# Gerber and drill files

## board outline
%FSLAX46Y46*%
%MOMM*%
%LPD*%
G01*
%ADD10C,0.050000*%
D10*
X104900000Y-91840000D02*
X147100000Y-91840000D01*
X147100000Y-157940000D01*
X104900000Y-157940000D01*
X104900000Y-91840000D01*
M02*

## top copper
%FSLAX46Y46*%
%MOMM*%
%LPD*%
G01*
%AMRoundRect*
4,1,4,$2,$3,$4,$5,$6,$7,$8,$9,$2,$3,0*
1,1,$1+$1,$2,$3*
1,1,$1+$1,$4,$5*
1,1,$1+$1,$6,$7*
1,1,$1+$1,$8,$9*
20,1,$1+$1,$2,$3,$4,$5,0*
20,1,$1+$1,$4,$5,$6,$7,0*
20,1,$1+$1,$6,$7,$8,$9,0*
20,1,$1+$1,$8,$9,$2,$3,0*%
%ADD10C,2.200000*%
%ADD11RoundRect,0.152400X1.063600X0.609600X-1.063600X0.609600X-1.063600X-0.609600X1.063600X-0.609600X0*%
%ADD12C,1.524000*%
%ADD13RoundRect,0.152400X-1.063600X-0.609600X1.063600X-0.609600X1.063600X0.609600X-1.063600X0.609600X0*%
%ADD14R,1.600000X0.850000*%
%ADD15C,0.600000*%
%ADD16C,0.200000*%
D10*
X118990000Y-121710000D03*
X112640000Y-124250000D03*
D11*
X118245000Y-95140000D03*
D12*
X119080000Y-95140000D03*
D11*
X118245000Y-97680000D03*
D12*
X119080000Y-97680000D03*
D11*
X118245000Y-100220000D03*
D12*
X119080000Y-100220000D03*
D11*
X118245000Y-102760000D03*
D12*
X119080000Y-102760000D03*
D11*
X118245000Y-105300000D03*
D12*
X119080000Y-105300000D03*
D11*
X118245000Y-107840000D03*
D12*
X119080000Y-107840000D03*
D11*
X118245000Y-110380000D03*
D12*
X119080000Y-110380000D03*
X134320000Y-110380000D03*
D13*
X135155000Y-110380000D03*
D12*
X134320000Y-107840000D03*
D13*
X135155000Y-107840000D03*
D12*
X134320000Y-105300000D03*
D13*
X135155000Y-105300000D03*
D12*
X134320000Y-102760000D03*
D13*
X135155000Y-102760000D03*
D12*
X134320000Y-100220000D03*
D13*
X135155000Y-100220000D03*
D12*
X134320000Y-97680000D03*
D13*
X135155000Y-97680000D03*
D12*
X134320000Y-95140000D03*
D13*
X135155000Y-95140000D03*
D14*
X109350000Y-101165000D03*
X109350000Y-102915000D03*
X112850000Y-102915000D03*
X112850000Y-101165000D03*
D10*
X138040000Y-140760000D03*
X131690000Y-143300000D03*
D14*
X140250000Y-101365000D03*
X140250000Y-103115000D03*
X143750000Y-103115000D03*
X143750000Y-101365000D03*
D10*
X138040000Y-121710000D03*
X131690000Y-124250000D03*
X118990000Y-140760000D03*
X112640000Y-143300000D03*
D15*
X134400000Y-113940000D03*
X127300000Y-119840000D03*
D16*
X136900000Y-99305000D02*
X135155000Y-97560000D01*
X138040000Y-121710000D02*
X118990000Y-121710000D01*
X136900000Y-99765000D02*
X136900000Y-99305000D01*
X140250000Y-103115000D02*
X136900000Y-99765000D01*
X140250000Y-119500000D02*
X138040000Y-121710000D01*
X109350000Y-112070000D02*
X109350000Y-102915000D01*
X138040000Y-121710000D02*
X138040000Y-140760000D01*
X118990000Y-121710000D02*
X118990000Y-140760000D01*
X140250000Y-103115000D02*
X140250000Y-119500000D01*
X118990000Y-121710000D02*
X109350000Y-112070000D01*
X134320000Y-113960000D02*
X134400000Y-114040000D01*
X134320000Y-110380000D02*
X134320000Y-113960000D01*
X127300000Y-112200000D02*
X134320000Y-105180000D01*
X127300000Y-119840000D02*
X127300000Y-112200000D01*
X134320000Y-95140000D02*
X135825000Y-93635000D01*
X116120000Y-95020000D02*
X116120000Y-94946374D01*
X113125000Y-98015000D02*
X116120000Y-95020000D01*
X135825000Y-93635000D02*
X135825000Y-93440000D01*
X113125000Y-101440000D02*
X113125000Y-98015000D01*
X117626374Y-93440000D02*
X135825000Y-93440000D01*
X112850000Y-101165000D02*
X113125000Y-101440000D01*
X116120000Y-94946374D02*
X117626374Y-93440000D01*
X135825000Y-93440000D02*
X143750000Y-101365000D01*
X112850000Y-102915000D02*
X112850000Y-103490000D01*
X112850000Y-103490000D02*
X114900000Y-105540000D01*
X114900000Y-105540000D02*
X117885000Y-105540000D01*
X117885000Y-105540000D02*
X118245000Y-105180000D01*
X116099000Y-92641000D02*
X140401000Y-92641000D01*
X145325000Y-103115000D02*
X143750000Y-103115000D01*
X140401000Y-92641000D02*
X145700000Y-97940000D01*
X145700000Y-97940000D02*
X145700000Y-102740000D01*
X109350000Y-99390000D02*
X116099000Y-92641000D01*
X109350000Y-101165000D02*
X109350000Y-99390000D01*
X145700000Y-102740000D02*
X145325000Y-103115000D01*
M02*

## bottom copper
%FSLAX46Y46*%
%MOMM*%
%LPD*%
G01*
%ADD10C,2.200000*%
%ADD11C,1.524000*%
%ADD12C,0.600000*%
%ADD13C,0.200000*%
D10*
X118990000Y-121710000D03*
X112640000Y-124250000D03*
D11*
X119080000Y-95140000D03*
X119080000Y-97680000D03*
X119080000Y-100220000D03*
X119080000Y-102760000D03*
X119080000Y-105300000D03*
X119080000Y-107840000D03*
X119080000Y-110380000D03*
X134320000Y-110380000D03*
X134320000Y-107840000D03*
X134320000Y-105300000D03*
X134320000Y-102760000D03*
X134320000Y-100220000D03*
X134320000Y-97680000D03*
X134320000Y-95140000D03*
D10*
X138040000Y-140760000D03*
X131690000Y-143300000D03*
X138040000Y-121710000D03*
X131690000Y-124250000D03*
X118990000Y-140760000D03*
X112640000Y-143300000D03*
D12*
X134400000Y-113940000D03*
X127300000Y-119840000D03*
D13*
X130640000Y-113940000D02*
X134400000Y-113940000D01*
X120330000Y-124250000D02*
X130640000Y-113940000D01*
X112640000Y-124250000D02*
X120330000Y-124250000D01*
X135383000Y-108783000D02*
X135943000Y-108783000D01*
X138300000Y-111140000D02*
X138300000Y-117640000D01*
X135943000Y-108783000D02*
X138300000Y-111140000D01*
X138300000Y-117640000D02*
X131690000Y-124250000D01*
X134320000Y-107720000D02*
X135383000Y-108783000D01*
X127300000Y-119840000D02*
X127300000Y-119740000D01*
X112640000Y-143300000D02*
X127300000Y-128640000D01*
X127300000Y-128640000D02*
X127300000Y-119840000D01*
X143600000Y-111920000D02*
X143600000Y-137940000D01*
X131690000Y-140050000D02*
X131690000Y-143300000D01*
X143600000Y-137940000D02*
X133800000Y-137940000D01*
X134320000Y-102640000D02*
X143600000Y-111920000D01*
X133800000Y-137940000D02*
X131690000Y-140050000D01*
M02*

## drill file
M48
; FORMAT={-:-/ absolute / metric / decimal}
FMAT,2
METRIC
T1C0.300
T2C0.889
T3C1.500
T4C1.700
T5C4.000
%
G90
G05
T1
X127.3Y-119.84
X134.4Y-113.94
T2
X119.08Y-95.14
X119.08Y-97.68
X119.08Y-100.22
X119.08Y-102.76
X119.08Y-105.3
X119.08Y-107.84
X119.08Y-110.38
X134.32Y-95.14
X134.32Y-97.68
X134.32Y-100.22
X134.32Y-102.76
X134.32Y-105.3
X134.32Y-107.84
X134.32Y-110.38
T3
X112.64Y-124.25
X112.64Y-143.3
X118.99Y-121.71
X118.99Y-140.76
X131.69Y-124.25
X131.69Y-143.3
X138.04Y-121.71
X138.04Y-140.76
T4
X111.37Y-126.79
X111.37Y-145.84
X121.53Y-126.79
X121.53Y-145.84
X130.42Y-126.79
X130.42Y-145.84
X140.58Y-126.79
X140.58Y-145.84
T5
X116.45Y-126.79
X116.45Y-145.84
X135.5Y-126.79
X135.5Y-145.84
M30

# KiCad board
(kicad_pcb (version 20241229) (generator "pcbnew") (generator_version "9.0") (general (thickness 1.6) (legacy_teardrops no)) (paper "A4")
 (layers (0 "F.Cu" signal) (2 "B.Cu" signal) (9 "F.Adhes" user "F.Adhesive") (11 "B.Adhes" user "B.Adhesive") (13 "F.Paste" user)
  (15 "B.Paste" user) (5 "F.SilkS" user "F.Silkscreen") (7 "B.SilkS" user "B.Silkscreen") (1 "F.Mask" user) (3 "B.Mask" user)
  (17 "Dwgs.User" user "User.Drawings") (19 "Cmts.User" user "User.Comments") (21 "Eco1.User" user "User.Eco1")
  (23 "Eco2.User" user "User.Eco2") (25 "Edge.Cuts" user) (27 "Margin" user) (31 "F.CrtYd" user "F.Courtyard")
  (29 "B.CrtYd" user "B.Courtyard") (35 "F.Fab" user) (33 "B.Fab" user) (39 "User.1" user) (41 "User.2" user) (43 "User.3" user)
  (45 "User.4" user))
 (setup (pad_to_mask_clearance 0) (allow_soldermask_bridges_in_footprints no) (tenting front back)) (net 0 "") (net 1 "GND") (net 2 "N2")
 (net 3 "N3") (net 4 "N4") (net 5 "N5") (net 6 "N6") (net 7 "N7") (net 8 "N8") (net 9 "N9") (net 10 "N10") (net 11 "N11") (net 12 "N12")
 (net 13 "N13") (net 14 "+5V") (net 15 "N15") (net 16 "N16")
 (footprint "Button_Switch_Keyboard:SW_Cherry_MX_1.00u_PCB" (layer "F.Cu") (at 118.99 121.71)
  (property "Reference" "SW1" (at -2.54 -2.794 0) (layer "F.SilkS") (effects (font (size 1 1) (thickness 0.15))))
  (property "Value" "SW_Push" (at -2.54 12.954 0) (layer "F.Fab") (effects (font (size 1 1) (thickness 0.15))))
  (pad "" np_thru_hole circle (at -7.62 5.08) (size 1.7 1.7) (drill 1.7) (layers "*.Cu" "*.Mask"))
  (pad "" np_thru_hole circle (at -2.54 5.08) (size 4 4) (drill 4) (layers "*.Cu" "*.Mask"))
  (pad "" np_thru_hole circle (at 2.54 5.08) (size 1.7 1.7) (drill 1.7) (layers "*.Cu" "*.Mask"))
  (pad "1" thru_hole circle (at 0 0) (size 2.2 2.2) (drill 1.5) (layers "*.Cu" "*.Mask") (remove_unused_layers no) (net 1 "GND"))
  (pad "2" thru_hole circle (at -6.35 2.54) (size 2.2 2.2) (drill 1.5) (layers "*.Cu" "*.Mask") (remove_unused_layers no) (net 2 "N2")))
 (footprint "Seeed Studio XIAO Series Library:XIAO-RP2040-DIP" (layer "F.Cu") (at 126.7 102.76)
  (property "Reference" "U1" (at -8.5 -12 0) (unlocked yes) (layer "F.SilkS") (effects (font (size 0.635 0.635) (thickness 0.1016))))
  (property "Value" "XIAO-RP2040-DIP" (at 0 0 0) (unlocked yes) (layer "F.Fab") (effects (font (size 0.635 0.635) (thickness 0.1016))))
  (pad "1" smd roundrect (at -8.455 -7.62 180) (size 2.432 1.524) (layers "F.Cu" "F.Mask") (roundrect_rratio 0.1) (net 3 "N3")
   (thermal_bridge_angle 45))
  (pad "1" thru_hole circle (at -7.62 -7.62 180) (size 1.524 1.524) (drill 0.889) (layers "*.Cu" "*.Mask") (remove_unused_layers no)
   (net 3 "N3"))
  (pad "2" smd roundrect (at -8.455 -5.08 180) (size 2.432 1.524) (layers "F.Cu" "F.Mask") (roundrect_rratio 0.1) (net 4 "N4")
   (thermal_bridge_angle 45))
  (pad "2" thru_hole circle (at -7.62 -5.08 180) (size 1.524 1.524) (drill 0.889) (layers "*.Cu" "*.Mask") (remove_unused_layers no)
   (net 4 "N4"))
  (pad "3" smd roundrect (at -8.455 -2.54 180) (size 2.432 1.524) (layers "F.Cu" "F.Mask") (roundrect_rratio 0.1) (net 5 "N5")
   (thermal_bridge_angle 45))
  (pad "3" thru_hole circle (at -7.62 -2.54 180) (size 1.524 1.524) (drill 0.889) (layers "*.Cu" "*.Mask") (remove_unused_layers no)
   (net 5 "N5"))
  (pad "4" smd roundrect (at -8.455 0 180) (size 2.432 1.524) (layers "F.Cu" "F.Mask") (roundrect_rratio 0.1) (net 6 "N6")
   (thermal_bridge_angle 45))
  (pad "4" thru_hole circle (at -7.62 0 180) (size 1.524 1.524) (drill 0.889) (layers "*.Cu" "*.Mask") (remove_unused_layers no)
   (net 6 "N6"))
  (pad "5" smd roundrect (at -8.455 2.54 180) (size 2.432 1.524) (layers "F.Cu" "F.Mask") (roundrect_rratio 0.1) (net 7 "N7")
   (thermal_bridge_angle 45))
  (pad "5" thru_hole circle (at -7.62 2.54 180) (size 1.524 1.524) (drill 0.889) (layers "*.Cu" "*.Mask") (remove_unused_layers no)
   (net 7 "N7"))
  (pad "6" smd roundrect (at -8.455 5.08 180) (size 2.432 1.524) (layers "F.Cu" "F.Mask") (roundrect_rratio 0.1) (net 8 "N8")
   (thermal_bridge_angle 45))
  (pad "6" thru_hole circle (at -7.62 5.08 180) (size 1.524 1.524) (drill 0.889) (layers "*.Cu" "*.Mask") (remove_unused_layers no)
   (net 8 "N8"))
  (pad "7" smd roundrect (at -8.455 7.62 180) (size 2.432 1.524) (layers "F.Cu" "F.Mask") (roundrect_rratio 0.1) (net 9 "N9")
   (thermal_bridge_angle 45))
  (pad "7" thru_hole circle (at -7.62 7.62 180) (size 1.524 1.524) (drill 0.889) (layers "*.Cu" "*.Mask") (remove_unused_layers no)
   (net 9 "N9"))
  (pad "8" thru_hole circle (at 7.62 7.62) (size 1.524 1.524) (drill 0.889) (layers "*.Cu" "*.Mask") (remove_unused_layers no) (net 2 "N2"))
  (pad "8" smd roundrect (at 8.455 7.62) (size 2.432 1.524) (layers "F.Cu" "F.Mask") (roundrect_rratio 0.1) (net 2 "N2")
   (thermal_bridge_angle 45))
  (pad "9" thru_hole circle (at 7.62 5.08) (size 1.524 1.524) (drill 0.889) (layers "*.Cu" "*.Mask") (remove_unused_layers no)
   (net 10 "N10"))
  (pad "9" smd roundrect (at 8.455 5.08) (size 2.432 1.524) (layers "F.Cu" "F.Mask") (roundrect_rratio 0.1) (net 10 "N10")
   (thermal_bridge_angle 45))
  (pad "10" thru_hole circle (at 7.62 2.54) (size 1.524 1.524) (drill 0.889) (layers "*.Cu" "*.Mask") (remove_unused_layers no)
   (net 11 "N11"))
  (pad "10" smd roundrect (at 8.455 2.54) (size 2.432 1.524) (layers "F.Cu" "F.Mask") (roundrect_rratio 0.1) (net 11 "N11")
   (thermal_bridge_angle 45))
  (pad "11" thru_hole circle (at 7.62 0) (size 1.524 1.524) (drill 0.889) (layers "*.Cu" "*.Mask") (remove_unused_layers no) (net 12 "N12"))
  (pad "11" smd roundrect (at 8.455 0) (size 2.432 1.524) (layers "F.Cu" "F.Mask") (roundrect_rratio 0.1) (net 12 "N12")
   (thermal_bridge_angle 45))
  (pad "12" thru_hole circle (at 7.62 -2.54) (size 1.524 1.524) (drill 0.889) (layers "*.Cu" "*.Mask") (remove_unused_layers no)
   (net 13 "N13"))
  (pad "12" smd roundrect (at 8.455 -2.54) (size 2.432 1.524) (layers "F.Cu" "F.Mask") (roundrect_rratio 0.1) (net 13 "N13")
   (thermal_bridge_angle 45))
  (pad "13" thru_hole circle (at 7.62 -5.08) (size 1.524 1.524) (drill 0.889) (layers "*.Cu" "*.Mask") (remove_unused_layers no)
   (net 1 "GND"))
  (pad "13" smd roundrect (at 8.455 -5.08) (size 2.432 1.524) (layers "F.Cu" "F.Mask") (roundrect_rratio 0.1) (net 1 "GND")
   (thermal_bridge_angle 45))
  (pad "14" thru_hole circle (at 7.62 -7.62) (size 1.524 1.524) (drill 0.889) (layers "*.Cu" "*.Mask") (remove_unused_layers no)
   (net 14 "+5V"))
  (pad "14" smd roundrect (at 8.455 -7.62) (size 2.432 1.524) (layers "F.Cu" "F.Mask") (roundrect_rratio 0.1) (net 14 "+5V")
   (thermal_bridge_angle 45)))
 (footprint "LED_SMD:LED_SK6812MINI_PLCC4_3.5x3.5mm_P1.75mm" (layer "F.Cu") (at 111.1 102.04)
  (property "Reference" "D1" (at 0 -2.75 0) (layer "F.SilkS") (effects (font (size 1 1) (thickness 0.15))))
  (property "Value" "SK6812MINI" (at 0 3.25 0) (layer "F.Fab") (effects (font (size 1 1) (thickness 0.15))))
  (pad "1" smd rect (at -1.75 -0.875) (size 1.6 0.85) (layers "F.Cu" "F.Mask" "F.Paste") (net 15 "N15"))
  (pad "2" smd rect (at -1.75 0.875) (size 1.6 0.85) (layers "F.Cu" "F.Mask" "F.Paste") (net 1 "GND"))
  (pad "3" smd rect (at 1.75 0.875) (size 1.6 0.85) (layers "F.Cu" "F.Mask" "F.Paste") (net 7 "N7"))
  (pad "4" smd rect (at 1.75 -0.875) (size 1.6 0.85) (layers "F.Cu" "F.Mask" "F.Paste") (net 14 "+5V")))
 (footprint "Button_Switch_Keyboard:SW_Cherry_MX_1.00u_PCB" (layer "F.Cu") (at 138.04 140.76)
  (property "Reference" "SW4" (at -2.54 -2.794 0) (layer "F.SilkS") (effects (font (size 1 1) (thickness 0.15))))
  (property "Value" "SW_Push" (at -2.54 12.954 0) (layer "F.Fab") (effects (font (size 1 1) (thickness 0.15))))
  (pad "" np_thru_hole circle (at -7.62 5.08) (size 1.7 1.7) (drill 1.7) (layers "*.Cu" "*.Mask"))
  (pad "" np_thru_hole circle (at -2.54 5.08) (size 4 4) (drill 4) (layers "*.Cu" "*.Mask"))
  (pad "" np_thru_hole circle (at 2.54 5.08) (size 1.7 1.7) (drill 1.7) (layers "*.Cu" "*.Mask"))
  (pad "1" thru_hole circle (at 0 0) (size 2.2 2.2) (drill 1.5) (layers "*.Cu" "*.Mask") (remove_unused_layers no) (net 1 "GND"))
  (pad "2" thru_hole circle (at -6.35 2.54) (size 2.2 2.2) (drill 1.5) (layers "*.Cu" "*.Mask") (remove_unused_layers no) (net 12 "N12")))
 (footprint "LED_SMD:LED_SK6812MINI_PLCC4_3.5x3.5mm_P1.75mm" (layer "F.Cu") (at 142 102.24)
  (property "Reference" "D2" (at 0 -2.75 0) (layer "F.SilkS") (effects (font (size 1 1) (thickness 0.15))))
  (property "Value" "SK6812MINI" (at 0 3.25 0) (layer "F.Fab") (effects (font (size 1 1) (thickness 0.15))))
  (pad "1" smd rect (at -1.75 -0.875) (size 1.6 0.85) (layers "F.Cu" "F.Mask" "F.Paste") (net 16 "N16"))
  (pad "2" smd rect (at -1.75 0.875) (size 1.6 0.85) (layers "F.Cu" "F.Mask" "F.Paste") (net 1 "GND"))
  (pad "3" smd rect (at 1.75 0.875) (size 1.6 0.85) (layers "F.Cu" "F.Mask" "F.Paste") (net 15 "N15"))
  (pad "4" smd rect (at 1.75 -0.875) (size 1.6 0.85) (layers "F.Cu" "F.Mask" "F.Paste") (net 14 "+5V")))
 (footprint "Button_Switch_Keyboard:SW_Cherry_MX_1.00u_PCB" (layer "F.Cu") (at 138.04 121.71)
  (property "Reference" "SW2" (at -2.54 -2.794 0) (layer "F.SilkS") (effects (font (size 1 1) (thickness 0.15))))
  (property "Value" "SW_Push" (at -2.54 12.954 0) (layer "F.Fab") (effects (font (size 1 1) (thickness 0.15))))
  (pad "" np_thru_hole circle (at -7.62 5.08) (size 1.7 1.7) (drill 1.7) (layers "*.Cu" "*.Mask"))
  (pad "" np_thru_hole circle (at -2.54 5.08) (size 4 4) (drill 4) (layers "*.Cu" "*.Mask"))
  (pad "" np_thru_hole circle (at 2.54 5.08) (size 1.7 1.7) (drill 1.7) (layers "*.Cu" "*.Mask"))
  (pad "1" thru_hole circle (at 0 0) (size 2.2 2.2) (drill 1.5) (layers "*.Cu" "*.Mask") (remove_unused_layers no) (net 1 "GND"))
  (pad "2" thru_hole circle (at -6.35 2.54) (size 2.2 2.2) (drill 1.5) (layers "*.Cu" "*.Mask") (remove_unused_layers no) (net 10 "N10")))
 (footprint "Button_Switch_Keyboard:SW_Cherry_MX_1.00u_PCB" (layer "F.Cu") (at 118.99 140.76)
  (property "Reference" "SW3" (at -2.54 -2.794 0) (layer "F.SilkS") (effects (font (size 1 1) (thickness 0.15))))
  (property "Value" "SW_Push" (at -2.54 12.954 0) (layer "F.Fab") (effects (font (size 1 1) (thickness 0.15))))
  (pad "" np_thru_hole circle (at -7.62 5.08) (size 1.7 1.7) (drill 1.7) (layers "*.Cu" "*.Mask"))
  (pad "" np_thru_hole circle (at -2.54 5.08) (size 4 4) (drill 4) (layers "*.Cu" "*.Mask"))
  (pad "" np_thru_hole circle (at 2.54 5.08) (size 1.7 1.7) (drill 1.7) (layers "*.Cu" "*.Mask"))
  (pad "1" thru_hole circle (at 0 0) (size 2.2 2.2) (drill 1.5) (layers "*.Cu" "*.Mask") (remove_unused_layers no) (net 1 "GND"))
  (pad "2" thru_hole circle (at -6.35 2.54) (size 2.2 2.2) (drill 1.5) (layers "*.Cu" "*.Mask") (remove_unused_layers no) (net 11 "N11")))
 (gr_rect (start 104.9 91.84) (end 147.1 157.94) (stroke (width 0.05) (type default)) (fill no) (layer "Edge.Cuts"))
 (segment (start 136.9 99.305) (end 135.155 97.56) (width 0.2) (layer "F.Cu") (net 1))
 (segment (start 138.04 121.71) (end 118.99 121.71) (width 0.2) (layer "F.Cu") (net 1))
 (segment (start 136.9 99.765) (end 136.9 99.305) (width 0.2) (layer "F.Cu") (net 1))
 (segment (start 140.25 103.115) (end 136.9 99.765) (width 0.2) (layer "F.Cu") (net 1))
 (segment (start 140.25 119.5) (end 138.04 121.71) (width 0.2) (layer "F.Cu") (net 1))
 (segment (start 109.35 112.07) (end 109.35 102.915) (width 0.2) (layer "F.Cu") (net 1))
 (segment (start 138.04 121.71) (end 138.04 140.76) (width 0.2) (layer "F.Cu") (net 1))
 (segment (start 118.99 121.71) (end 118.99 140.76) (width 0.2) (layer "F.Cu") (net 1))
 (segment (start 140.25 103.115) (end 140.25 119.5) (width 0.2) (layer "F.Cu") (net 1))
 (segment (start 118.99 121.71) (end 109.35 112.07) (width 0.2) (layer "F.Cu") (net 1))
 (segment (start 134.32 113.96) (end 134.4 114.04) (width 0.2) (layer "F.Cu") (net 2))
 (segment (start 134.32 110.38) (end 134.32 113.96) (width 0.2) (layer "F.Cu") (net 2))
 (via (at 134.4 113.94) (size 0.6) (drill 0.3) (layers "F.Cu" "B.Cu") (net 2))
 (segment (start 130.64 113.94) (end 134.4 113.94) (width 0.2) (layer "B.Cu") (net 2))
 (segment (start 120.33 124.25) (end 130.64 113.94) (width 0.2) (layer "B.Cu") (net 2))
 (segment (start 112.64 124.25) (end 120.33 124.25) (width 0.2) (layer "B.Cu") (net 2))
 (segment (start 135.383 108.783) (end 135.943 108.783) (width 0.2) (layer "B.Cu") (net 10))
 (segment (start 138.3 111.14) (end 138.3 117.64) (width 0.2) (layer "B.Cu") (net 10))
 (segment (start 135.943 108.783) (end 138.3 111.14) (width 0.2) (layer "B.Cu") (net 10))
 (segment (start 138.3 117.64) (end 131.69 124.25) (width 0.2) (layer "B.Cu") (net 10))
 (segment (start 134.32 107.72) (end 135.383 108.783) (width 0.2) (layer "B.Cu") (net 10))
 (segment (start 127.3 112.2) (end 134.32 105.18) (width 0.2) (layer "F.Cu") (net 11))
 (segment (start 127.3 119.84) (end 127.3 112.2) (width 0.2) (layer "F.Cu") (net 11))
 (via (at 127.3 119.84) (size 0.6) (drill 0.3) (layers "F.Cu" "B.Cu") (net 11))
 (segment (start 127.3 119.84) (end 127.3 119.74) (width 0.2) (layer "B.Cu") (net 11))
 (segment (start 112.64 143.3) (end 127.3 128.64) (width 0.2) (layer "B.Cu") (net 11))
 (segment (start 127.3 128.64) (end 127.3 119.84) (width 0.2) (layer "B.Cu") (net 11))
 (segment (start 143.6 111.92) (end 143.6 137.94) (width 0.2) (layer "B.Cu") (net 12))
 (segment (start 131.69 140.05) (end 131.69 143.3) (width 0.2) (layer "B.Cu") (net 12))
 (segment (start 143.6 137.94) (end 133.8 137.94) (width 0.2) (layer "B.Cu") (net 12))
 (segment (start 134.32 102.64) (end 143.6 111.92) (width 0.2) (layer "B.Cu") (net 12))
 (segment (start 133.8 137.94) (end 131.69 140.05) (width 0.2) (layer "B.Cu") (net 12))
 (segment (start 134.32 95.14) (end 135.825 93.635) (width 0.2) (layer "F.Cu") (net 14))
 (segment (start 116.12 95.02) (end 116.12 94.946374) (width 0.2) (layer "F.Cu") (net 14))
 (segment (start 113.125 98.015) (end 116.12 95.02) (width 0.2) (layer "F.Cu") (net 14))
 (segment (start 135.825 93.635) (end 135.825 93.44) (width 0.2) (layer "F.Cu") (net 14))
 (segment (start 113.125 101.44) (end 113.125 98.015) (width 0.2) (layer "F.Cu") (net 14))
 (segment (start 117.626374 93.44) (end 135.825 93.44) (width 0.2) (layer "F.Cu") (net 14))
 (segment (start 112.85 101.165) (end 113.125 101.44) (width 0.2) (layer "F.Cu") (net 14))
 (segment (start 116.12 94.946374) (end 117.626374 93.44) (width 0.2) (layer "F.Cu") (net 14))
 (segment (start 135.825 93.44) (end 143.75 101.365) (width 0.2) (layer "F.Cu") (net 14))
 (segment (start 112.85 102.915) (end 112.85 103.49) (width 0.2) (layer "F.Cu") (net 7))
 (segment (start 112.85 103.49) (end 114.9 105.54) (width 0.2) (layer "F.Cu") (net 7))
 (segment (start 114.9 105.54) (end 117.885 105.54) (width 0.2) (layer "F.Cu") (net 7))
 (segment (start 117.885 105.54) (end 118.245 105.18) (width 0.2) (layer "F.Cu") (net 7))
 (segment (start 116.099 92.641) (end 140.401 92.641) (width 0.2) (layer "F.Cu") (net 15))
 (segment (start 145.325 103.115) (end 143.75 103.115) (width 0.2) (layer "F.Cu") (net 15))
 (segment (start 140.401 92.641) (end 145.7 97.94) (width 0.2) (layer "F.Cu") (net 15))
 (segment (start 145.7 97.94) (end 145.7 102.74) (width 0.2) (layer "F.Cu") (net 15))
 (segment (start 109.35 99.39) (end 116.099 92.641) (width 0.2) (layer "F.Cu") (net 15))
 (segment (start 109.35 101.165) (end 109.35 99.39) (width 0.2) (layer "F.Cu") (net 15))
 (segment (start 145.7 102.74) (end 145.325 103.115) (width 0.2) (layer "F.Cu") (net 15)))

